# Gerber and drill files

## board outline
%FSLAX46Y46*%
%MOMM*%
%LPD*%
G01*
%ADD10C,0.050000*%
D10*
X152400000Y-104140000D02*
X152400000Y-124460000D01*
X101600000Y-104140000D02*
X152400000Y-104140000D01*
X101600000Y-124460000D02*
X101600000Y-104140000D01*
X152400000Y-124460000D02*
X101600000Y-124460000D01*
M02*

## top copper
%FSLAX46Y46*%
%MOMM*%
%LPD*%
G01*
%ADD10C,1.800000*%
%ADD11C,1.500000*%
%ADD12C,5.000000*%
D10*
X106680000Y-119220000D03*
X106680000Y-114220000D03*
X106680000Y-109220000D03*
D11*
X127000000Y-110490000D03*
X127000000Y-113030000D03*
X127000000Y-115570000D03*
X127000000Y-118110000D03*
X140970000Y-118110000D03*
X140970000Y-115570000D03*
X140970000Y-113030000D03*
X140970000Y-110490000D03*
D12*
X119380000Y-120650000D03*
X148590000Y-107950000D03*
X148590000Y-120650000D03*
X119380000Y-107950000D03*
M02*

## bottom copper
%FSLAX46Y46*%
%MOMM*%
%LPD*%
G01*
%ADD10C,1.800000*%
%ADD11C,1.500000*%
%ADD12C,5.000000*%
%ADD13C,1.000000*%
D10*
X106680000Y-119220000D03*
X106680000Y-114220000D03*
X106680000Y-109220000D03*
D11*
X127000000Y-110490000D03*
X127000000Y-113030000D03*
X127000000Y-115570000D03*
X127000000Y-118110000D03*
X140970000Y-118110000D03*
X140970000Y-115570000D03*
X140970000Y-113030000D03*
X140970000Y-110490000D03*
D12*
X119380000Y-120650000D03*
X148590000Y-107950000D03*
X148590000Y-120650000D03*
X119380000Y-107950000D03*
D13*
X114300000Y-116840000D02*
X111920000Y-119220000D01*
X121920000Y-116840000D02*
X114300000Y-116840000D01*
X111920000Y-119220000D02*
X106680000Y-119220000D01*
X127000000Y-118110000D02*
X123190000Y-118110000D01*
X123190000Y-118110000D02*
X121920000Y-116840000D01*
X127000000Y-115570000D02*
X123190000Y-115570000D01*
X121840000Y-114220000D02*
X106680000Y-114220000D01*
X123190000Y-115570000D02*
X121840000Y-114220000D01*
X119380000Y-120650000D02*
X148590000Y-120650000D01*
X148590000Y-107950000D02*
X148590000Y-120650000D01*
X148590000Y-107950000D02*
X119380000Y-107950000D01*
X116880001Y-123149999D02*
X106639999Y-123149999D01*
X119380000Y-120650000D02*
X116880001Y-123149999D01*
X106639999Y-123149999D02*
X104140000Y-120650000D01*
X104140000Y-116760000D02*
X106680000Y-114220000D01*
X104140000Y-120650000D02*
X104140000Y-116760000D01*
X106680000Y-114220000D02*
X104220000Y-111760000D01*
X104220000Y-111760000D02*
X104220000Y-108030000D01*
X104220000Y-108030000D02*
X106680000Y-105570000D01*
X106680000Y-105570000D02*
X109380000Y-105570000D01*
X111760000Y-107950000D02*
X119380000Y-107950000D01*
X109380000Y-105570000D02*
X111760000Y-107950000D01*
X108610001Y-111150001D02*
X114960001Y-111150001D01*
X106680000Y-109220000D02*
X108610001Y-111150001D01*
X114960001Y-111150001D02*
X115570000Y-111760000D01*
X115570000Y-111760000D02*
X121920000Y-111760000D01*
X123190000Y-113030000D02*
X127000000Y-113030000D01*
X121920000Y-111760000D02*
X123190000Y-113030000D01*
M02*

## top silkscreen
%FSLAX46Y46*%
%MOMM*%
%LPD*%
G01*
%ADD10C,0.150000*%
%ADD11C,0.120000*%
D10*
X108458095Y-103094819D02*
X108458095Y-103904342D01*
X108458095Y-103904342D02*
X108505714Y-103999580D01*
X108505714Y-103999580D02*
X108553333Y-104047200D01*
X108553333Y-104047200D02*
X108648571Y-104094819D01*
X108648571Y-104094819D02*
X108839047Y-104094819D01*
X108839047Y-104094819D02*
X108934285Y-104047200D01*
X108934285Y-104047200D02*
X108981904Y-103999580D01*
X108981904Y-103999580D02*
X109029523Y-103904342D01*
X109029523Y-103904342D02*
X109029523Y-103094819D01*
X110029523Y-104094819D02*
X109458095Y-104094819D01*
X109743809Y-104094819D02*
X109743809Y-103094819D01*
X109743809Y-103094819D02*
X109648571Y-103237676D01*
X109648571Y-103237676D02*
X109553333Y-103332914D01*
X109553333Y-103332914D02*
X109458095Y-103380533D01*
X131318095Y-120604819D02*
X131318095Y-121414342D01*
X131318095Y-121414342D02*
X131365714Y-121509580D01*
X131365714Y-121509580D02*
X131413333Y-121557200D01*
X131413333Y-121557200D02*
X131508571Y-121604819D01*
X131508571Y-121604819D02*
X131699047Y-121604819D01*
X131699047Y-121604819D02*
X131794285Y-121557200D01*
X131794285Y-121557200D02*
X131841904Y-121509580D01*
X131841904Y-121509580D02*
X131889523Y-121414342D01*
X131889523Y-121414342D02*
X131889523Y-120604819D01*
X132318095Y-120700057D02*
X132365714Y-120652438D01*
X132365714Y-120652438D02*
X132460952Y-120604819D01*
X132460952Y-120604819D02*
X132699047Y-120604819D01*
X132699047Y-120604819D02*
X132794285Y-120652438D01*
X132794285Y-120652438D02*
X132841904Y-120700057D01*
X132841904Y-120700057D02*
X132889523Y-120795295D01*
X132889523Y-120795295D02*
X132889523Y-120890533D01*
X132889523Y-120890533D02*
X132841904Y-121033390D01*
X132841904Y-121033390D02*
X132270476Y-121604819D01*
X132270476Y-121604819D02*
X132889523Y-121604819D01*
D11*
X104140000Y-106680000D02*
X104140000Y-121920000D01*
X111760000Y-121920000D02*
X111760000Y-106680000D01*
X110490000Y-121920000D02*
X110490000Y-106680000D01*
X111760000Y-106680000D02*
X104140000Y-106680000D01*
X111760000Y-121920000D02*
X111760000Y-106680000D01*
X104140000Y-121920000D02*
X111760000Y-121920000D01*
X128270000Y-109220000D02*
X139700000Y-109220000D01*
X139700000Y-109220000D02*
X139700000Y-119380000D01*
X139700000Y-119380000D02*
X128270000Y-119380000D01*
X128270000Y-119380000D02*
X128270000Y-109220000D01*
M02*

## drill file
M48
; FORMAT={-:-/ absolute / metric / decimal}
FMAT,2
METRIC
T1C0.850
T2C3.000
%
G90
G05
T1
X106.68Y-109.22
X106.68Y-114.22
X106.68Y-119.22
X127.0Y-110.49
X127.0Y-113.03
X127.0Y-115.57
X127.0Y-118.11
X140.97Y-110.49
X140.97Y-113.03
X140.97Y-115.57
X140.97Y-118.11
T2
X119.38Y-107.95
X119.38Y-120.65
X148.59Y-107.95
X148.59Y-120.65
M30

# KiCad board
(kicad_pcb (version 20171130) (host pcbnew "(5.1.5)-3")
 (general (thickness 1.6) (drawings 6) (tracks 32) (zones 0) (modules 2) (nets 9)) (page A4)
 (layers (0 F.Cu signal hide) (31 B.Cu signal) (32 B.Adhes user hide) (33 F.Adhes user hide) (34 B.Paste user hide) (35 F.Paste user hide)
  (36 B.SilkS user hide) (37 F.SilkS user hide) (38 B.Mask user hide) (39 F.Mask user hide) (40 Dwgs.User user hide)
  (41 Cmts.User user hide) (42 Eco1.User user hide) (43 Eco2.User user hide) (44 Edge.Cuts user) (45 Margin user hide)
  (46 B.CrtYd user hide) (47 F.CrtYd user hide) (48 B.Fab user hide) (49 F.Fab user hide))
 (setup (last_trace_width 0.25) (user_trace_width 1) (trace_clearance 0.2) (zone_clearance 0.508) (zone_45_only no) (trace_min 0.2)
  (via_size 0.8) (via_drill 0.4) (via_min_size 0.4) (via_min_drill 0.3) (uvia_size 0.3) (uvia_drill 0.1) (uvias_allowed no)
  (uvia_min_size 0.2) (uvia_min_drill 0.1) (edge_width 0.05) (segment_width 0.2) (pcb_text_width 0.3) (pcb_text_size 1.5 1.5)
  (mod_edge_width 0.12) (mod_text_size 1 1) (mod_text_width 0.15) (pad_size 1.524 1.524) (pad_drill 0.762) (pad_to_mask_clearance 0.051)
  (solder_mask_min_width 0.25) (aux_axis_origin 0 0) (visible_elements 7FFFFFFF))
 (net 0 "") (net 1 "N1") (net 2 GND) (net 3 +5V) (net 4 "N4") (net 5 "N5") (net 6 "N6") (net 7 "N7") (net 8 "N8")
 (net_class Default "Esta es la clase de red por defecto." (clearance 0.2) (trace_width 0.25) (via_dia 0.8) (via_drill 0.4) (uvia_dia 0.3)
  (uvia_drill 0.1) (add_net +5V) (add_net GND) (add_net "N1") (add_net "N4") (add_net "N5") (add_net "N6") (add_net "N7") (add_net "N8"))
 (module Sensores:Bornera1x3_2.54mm (layer F.Cu) (at 106.68 109.22 180)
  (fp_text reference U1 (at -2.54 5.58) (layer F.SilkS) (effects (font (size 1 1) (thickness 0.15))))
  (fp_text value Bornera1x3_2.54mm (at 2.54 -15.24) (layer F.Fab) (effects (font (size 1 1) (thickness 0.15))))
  (fp_line (start 2.54 2.54) (end 2.54 -12.7) (layer F.SilkS) (width 0.12))
  (fp_line (start -5.08 -12.7) (end -5.08 2.54) (layer F.SilkS) (width 0.12))
  (fp_line (start -3.81 -12.7) (end -3.81 2.54) (layer F.SilkS) (width 0.12))
  (fp_line (start -5.08 2.54) (end 2.54 2.54) (layer F.SilkS) (width 0.12))
  (fp_line (start -5.08 -12.7) (end -5.08 2.54) (layer F.SilkS) (width 0.12))
  (fp_line (start 2.54 -12.7) (end -5.08 -12.7) (layer F.SilkS) (width 0.12))
  (pad 3 thru_hole circle (at 0 -10 180) (size 1.8 1.8) (drill 0.85) (layers *.Cu *.Mask) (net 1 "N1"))
  (pad 2 thru_hole circle (at 0 -5 180) (size 1.8 1.8) (drill 0.85) (layers *.Cu *.Mask) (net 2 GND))
  (pad 1 thru_hole circle (at 0 0 180) (size 1.8 1.8) (drill 0.85) (layers *.Cu *.Mask) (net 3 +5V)))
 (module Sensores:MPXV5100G (layer F.Cu) (at 127 110.49)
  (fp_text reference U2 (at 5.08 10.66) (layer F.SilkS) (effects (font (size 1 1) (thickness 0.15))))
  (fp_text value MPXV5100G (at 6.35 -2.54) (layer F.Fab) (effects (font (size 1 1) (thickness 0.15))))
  (fp_line (start 1.27 -1.27) (end 12.7 -1.27) (layer F.SilkS) (width 0.12))
  (fp_line (start 12.7 -1.27) (end 12.7 8.89) (layer F.SilkS) (width 0.12))
  (fp_line (start 12.7 8.89) (end 1.27 8.89) (layer F.SilkS) (width 0.12))
  (fp_line (start 1.27 8.89) (end 1.27 -1.27) (layer F.SilkS) (width 0.12))
  (pad 1 thru_hole circle (at 0 0) (size 1.5 1.5) (drill 0.85) (layers *.Cu *.Mask) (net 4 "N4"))
  (pad 2 thru_hole circle (at 0 2.54) (size 1.5 1.5) (drill 0.85) (layers *.Cu *.Mask) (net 3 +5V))
  (pad 3 thru_hole circle (at 0 5.08) (size 1.5 1.5) (drill 0.85) (layers *.Cu *.Mask) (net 2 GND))
  (pad 4 thru_hole circle (at 0 7.62) (size 1.5 1.5) (drill 0.85) (layers *.Cu *.Mask) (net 1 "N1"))
  (pad 5 thru_hole circle (at 13.97 7.62) (size 1.5 1.5) (drill 0.85) (layers *.Cu *.Mask) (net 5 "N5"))
  (pad 6 thru_hole circle (at 13.97 5.08) (size 1.5 1.5) (drill 0.85) (layers *.Cu *.Mask) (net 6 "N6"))
  (pad 7 thru_hole circle (at 13.97 2.54) (size 1.5 1.5) (drill 0.85) (layers *.Cu *.Mask) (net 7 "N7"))
  (pad 8 thru_hole circle (at 13.97 0) (size 1.5 1.5) (drill 0.85) (layers *.Cu *.Mask) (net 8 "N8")))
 (gr_line (start 152.4 104.14) (end 152.4 124.46) (layer Edge.Cuts) (width 0.05))
 (gr_line (start 101.6 104.14) (end 152.4 104.14) (layer Edge.Cuts) (width 0.05))
 (gr_line (start 101.6 124.46) (end 101.6 104.14) (layer Edge.Cuts) (width 0.05))
 (gr_line (start 152.4 124.46) (end 101.6 124.46) (layer Edge.Cuts) (width 0.05))
 (segment (start 114.3 116.84) (end 111.92 119.22) (width 1) (layer B.Cu) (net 1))
 (segment (start 121.92 116.84) (end 114.3 116.84) (width 1) (layer B.Cu) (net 1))
 (segment (start 111.92 119.22) (end 106.68 119.22) (width 1) (layer B.Cu) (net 1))
 (segment (start 127 118.11) (end 123.19 118.11) (width 1) (layer B.Cu) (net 1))
 (segment (start 123.19 118.11) (end 121.92 116.84) (width 1) (layer B.Cu) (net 1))
 (segment (start 127 115.57) (end 123.19 115.57) (width 1) (layer B.Cu) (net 2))
 (segment (start 121.84 114.22) (end 106.68 114.22) (width 1) (layer B.Cu) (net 2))
 (segment (start 123.19 115.57) (end 121.84 114.22) (width 1) (layer B.Cu) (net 2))
 (segment (start 119.38 120.65) (end 148.59 120.65) (width 1) (layer B.Cu) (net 2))
 (segment (start 148.59 107.95) (end 148.59 120.65) (width 1) (layer B.Cu) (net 2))
 (via (at 119.38 120.65) (size 5) (drill 3) (layers F.Cu B.Cu) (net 2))
 (via (at 148.59 107.95) (size 5) (drill 3) (layers F.Cu B.Cu) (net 2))
 (via (at 148.59 120.65) (size 5) (drill 3) (layers F.Cu B.Cu) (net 2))
 (via (at 119.38 107.95) (size 5) (drill 3) (layers F.Cu B.Cu) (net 2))
 (segment (start 148.59 107.95) (end 119.38 107.95) (width 1) (layer B.Cu) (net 2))
 (segment (start 116.880001 123.149999) (end 106.639999 123.149999) (width 1) (layer B.Cu) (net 2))
 (segment (start 119.38 120.65) (end 116.880001 123.149999) (width 1) (layer B.Cu) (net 2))
 (segment (start 106.639999 123.149999) (end 104.14 120.65) (width 1) (layer B.Cu) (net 2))
 (segment (start 104.14 116.76) (end 106.68 114.22) (width 1) (layer B.Cu) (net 2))
 (segment (start 104.14 120.65) (end 104.14 116.76) (width 1) (layer B.Cu) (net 2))
 (segment (start 106.68 114.22) (end 104.22 111.76) (width 1) (layer B.Cu) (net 2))
 (segment (start 104.22 111.76) (end 104.22 108.03) (width 1) (layer B.Cu) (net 2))
 (segment (start 104.22 108.03) (end 106.68 105.57) (width 1) (layer B.Cu) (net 2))
 (segment (start 106.68 105.57) (end 109.38 105.57) (width 1) (layer B.Cu) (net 2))
 (segment (start 111.76 107.95) (end 119.38 107.95) (width 1) (layer B.Cu) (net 2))
 (segment (start 109.38 105.57) (end 111.76 107.95) (width 1) (layer B.Cu) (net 2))
 (segment (start 108.610001 111.150001) (end 114.960001 111.150001) (width 1) (layer B.Cu) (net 3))
 (segment (start 106.68 109.22) (end 108.610001 111.150001) (width 1) (layer B.Cu) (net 3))
 (segment (start 114.960001 111.150001) (end 115.57 111.76) (width 1) (layer B.Cu) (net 3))
 (segment (start 115.57 111.76) (end 121.92 111.76) (width 1) (layer B.Cu) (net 3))
 (segment (start 123.19 113.03) (end 127 113.03) (width 1) (layer B.Cu) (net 3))
 (segment (start 121.92 111.76) (end 123.19 113.03) (width 1) (layer B.Cu) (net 3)))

